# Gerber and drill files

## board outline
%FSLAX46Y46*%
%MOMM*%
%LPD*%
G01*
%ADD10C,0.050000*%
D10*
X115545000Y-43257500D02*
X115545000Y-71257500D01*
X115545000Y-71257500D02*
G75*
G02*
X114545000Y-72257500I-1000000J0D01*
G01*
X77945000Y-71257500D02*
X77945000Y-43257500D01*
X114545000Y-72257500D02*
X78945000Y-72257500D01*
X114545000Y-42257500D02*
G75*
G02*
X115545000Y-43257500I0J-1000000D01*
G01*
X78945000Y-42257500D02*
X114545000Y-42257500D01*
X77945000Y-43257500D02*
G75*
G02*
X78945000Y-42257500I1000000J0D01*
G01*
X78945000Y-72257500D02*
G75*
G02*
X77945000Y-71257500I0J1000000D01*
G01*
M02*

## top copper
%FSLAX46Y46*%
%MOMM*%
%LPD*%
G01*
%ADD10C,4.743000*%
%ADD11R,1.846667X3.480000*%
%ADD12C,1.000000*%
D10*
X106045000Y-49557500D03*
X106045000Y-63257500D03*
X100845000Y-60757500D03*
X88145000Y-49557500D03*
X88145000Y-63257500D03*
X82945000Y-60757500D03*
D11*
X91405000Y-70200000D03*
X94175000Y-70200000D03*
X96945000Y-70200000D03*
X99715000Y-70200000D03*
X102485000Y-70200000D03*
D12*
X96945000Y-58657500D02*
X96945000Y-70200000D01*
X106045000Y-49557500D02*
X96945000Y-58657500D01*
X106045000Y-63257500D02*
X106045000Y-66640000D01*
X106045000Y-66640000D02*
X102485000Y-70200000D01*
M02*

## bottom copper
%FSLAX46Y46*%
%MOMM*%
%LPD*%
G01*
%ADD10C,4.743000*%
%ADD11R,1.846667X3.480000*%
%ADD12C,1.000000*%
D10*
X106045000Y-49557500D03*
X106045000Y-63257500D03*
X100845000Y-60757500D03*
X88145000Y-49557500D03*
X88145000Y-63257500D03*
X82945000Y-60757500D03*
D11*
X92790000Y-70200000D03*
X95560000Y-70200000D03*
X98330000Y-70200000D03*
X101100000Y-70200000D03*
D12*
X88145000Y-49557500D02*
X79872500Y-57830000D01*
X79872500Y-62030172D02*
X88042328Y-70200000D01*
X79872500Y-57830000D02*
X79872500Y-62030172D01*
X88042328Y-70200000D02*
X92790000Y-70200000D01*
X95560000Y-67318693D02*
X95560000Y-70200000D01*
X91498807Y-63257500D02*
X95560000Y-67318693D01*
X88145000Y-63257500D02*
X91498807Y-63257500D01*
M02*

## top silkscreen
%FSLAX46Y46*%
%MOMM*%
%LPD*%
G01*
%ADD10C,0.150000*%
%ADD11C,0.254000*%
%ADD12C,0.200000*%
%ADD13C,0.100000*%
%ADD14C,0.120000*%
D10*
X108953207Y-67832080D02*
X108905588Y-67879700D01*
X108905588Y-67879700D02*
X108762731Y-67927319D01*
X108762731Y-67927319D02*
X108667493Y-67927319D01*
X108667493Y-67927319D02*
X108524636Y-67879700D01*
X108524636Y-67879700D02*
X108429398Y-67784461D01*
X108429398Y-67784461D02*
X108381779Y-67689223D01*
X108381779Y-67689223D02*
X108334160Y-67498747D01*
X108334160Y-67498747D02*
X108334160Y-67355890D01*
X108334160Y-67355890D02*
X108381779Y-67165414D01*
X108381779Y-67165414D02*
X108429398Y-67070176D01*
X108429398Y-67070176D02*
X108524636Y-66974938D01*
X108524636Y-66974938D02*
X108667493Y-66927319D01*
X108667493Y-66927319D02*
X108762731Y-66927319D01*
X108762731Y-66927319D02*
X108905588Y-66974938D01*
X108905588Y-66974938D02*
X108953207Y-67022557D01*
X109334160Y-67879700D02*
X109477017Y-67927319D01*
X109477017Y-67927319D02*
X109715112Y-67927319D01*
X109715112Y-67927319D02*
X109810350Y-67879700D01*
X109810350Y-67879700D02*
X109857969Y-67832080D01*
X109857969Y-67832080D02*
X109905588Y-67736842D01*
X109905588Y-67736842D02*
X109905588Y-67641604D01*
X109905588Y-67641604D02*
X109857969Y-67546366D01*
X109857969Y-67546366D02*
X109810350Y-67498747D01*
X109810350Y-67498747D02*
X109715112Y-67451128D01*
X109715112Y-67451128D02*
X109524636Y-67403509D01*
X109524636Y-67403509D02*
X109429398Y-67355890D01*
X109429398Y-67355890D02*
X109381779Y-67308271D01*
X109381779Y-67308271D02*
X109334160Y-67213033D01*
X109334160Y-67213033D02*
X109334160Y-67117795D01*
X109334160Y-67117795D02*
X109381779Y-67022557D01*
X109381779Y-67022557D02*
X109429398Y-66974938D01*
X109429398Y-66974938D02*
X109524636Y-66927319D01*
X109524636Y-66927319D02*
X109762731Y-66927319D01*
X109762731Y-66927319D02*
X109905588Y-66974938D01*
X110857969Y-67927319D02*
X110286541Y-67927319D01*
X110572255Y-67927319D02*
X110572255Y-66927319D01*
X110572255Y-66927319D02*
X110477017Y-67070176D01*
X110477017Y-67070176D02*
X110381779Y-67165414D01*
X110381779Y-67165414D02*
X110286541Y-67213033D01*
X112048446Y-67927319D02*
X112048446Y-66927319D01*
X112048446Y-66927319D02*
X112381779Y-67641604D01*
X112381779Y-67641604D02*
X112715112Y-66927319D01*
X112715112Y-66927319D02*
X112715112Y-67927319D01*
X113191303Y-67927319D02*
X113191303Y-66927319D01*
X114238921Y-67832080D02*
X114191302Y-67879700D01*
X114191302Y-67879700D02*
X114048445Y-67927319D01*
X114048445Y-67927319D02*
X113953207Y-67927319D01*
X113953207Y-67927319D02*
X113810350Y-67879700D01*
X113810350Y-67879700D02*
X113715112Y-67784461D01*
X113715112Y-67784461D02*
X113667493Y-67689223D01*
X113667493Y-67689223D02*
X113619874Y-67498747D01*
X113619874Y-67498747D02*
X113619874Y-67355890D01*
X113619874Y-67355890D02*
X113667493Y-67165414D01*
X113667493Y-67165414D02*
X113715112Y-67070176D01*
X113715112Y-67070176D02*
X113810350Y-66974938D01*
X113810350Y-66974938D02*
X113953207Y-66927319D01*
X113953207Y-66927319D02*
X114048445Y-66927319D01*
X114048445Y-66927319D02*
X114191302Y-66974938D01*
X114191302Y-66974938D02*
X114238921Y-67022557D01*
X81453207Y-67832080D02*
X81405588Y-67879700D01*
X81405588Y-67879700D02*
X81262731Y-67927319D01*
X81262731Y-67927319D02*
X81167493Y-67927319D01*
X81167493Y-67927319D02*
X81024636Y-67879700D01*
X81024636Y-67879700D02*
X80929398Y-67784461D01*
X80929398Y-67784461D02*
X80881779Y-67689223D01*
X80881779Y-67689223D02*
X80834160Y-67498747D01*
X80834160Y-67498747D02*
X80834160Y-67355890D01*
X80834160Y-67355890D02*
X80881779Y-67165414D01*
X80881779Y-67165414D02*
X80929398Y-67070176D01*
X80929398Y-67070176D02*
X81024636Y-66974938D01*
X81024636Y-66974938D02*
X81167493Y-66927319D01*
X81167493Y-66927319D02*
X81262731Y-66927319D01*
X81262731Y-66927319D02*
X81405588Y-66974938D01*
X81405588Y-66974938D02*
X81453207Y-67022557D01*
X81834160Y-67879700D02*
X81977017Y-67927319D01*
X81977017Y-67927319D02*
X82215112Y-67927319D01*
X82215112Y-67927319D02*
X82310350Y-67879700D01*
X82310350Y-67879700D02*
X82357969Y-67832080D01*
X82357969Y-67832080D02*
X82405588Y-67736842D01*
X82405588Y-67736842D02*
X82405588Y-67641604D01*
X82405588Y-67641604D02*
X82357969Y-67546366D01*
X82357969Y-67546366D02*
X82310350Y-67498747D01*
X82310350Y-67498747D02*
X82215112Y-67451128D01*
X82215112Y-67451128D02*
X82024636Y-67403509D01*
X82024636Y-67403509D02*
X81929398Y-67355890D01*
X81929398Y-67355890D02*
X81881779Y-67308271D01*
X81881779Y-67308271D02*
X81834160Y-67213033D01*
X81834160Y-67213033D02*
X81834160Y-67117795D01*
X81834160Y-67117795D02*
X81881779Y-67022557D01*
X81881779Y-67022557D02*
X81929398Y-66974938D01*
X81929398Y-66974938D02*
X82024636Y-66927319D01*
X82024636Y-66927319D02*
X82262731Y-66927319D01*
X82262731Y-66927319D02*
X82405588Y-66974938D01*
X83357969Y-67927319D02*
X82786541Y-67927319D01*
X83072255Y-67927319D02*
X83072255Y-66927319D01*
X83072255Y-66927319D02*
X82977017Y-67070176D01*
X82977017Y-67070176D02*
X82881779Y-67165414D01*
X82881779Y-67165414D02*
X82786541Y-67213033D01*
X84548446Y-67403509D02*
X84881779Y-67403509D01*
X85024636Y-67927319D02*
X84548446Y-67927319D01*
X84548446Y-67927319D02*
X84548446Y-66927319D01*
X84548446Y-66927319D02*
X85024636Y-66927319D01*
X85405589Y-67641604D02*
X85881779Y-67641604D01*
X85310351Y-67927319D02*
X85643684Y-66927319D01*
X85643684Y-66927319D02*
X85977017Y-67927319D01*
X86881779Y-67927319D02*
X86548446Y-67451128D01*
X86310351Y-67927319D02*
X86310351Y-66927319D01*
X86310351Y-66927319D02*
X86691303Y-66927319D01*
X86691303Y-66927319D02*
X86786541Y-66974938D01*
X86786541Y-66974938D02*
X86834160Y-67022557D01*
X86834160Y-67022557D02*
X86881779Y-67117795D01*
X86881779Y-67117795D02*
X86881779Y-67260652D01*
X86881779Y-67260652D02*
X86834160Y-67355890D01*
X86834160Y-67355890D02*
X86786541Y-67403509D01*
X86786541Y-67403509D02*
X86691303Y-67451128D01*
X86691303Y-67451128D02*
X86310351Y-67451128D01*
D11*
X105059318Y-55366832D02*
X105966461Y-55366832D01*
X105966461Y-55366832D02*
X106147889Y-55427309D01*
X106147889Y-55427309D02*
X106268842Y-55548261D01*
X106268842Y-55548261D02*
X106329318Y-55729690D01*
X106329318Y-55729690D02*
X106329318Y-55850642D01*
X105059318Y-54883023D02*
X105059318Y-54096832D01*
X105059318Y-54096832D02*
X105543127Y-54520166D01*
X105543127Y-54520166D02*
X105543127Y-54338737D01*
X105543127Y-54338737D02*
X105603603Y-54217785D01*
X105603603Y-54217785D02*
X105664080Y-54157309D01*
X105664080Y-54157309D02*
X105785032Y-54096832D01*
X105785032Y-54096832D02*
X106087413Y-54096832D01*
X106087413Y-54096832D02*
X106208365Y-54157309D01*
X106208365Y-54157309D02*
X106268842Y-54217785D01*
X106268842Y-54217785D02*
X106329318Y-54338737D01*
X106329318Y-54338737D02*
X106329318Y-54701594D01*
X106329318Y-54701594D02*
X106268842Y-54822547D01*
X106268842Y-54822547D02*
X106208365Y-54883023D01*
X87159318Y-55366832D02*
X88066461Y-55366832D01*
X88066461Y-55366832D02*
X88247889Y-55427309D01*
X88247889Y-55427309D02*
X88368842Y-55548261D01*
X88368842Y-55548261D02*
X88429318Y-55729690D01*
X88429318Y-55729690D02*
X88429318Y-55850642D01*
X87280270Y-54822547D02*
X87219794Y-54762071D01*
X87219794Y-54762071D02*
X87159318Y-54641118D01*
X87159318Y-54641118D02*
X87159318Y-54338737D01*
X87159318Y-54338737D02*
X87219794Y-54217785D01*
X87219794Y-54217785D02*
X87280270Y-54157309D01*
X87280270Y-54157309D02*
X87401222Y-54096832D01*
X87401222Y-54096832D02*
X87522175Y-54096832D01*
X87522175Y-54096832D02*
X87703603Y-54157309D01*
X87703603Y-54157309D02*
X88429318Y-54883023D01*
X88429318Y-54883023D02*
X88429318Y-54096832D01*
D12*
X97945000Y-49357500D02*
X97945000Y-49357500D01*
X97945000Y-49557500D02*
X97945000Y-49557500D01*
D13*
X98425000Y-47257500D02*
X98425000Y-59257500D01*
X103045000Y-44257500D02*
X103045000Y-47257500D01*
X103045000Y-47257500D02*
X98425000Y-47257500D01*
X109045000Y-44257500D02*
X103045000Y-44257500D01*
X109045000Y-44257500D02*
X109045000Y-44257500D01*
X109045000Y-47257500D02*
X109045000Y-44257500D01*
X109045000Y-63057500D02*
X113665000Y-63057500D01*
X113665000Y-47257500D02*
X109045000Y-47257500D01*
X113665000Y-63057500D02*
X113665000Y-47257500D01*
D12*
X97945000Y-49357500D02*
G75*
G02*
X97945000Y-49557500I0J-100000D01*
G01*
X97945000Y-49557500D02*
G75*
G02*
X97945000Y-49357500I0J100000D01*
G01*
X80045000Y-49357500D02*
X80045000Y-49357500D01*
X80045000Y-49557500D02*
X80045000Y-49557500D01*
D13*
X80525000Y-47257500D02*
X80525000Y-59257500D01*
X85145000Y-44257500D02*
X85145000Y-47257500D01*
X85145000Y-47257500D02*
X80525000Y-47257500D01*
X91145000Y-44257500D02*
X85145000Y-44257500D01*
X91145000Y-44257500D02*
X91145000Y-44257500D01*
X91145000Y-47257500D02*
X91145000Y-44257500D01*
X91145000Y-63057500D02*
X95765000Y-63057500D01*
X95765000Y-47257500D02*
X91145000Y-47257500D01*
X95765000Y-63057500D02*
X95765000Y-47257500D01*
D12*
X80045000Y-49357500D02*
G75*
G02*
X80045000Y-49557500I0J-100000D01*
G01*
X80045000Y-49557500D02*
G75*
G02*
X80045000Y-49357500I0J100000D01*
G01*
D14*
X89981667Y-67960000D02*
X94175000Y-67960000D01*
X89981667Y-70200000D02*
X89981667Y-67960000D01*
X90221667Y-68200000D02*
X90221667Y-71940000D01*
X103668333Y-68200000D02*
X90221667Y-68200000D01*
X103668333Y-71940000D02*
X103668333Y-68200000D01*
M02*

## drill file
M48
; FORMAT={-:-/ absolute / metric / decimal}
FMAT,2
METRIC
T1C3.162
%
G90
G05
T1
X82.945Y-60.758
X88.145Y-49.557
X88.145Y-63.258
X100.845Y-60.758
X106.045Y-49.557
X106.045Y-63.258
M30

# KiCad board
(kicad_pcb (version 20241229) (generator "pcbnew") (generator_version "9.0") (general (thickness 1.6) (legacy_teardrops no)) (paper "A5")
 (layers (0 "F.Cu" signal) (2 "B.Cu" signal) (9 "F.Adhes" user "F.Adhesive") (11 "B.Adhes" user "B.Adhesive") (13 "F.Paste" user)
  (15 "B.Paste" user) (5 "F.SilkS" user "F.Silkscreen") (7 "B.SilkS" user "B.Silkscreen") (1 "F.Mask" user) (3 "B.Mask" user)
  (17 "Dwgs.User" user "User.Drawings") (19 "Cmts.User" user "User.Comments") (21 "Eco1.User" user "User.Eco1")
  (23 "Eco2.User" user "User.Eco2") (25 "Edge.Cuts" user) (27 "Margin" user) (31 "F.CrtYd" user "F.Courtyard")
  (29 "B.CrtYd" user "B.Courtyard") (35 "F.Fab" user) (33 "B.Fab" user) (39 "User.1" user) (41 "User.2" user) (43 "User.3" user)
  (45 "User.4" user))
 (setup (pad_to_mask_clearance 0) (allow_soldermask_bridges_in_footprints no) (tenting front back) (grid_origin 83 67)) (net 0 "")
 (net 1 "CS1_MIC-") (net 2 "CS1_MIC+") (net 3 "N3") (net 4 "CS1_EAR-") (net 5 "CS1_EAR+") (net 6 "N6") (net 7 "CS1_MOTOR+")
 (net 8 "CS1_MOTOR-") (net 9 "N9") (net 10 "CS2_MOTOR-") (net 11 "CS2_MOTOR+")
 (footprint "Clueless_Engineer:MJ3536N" (layer "F.Cu") (at 105.755 54.9435 -90)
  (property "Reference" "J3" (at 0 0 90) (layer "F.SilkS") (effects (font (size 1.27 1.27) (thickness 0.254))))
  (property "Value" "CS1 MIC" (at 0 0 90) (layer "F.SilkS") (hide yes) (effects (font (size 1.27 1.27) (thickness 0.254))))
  (fp_line (start -5.586 7.81) (end -5.586 7.81) (stroke (width 0.2) (type solid)) (layer "F.SilkS"))
  (fp_line (start -5.386 7.81) (end -5.386 7.81) (stroke (width 0.2) (type solid)) (layer "F.SilkS"))
  (fp_line (start -7.686 7.33) (end 4.314 7.33) (stroke (width 0.1) (type solid)) (layer "F.SilkS"))
  (fp_line (start -10.686 2.71) (end -7.686 2.71) (stroke (width 0.1) (type solid)) (layer "F.SilkS"))
  (fp_line (start -7.686 2.71) (end -7.686 7.33) (stroke (width 0.1) (type solid)) (layer "F.SilkS"))
  (fp_line (start -10.686 -3.29) (end -10.686 2.71) (stroke (width 0.1) (type solid)) (layer "F.SilkS"))
  (fp_line (start -10.686 -3.29) (end -10.686 -3.29) (stroke (width 0.1) (type solid)) (layer "F.SilkS"))
  (fp_line (start -7.686 -3.29) (end -10.686 -3.29) (stroke (width 0.1) (type solid)) (layer "F.SilkS"))
  (fp_line (start 8.114 -3.29) (end 8.114 -7.91) (stroke (width 0.1) (type solid)) (layer "F.SilkS"))
  (fp_line (start -7.686 -7.91) (end -7.686 -3.29) (stroke (width 0.1) (type solid)) (layer "F.SilkS"))
  (fp_line (start 8.114 -7.91) (end -7.686 -7.91) (stroke (width 0.1) (type solid)) (layer "F.SilkS"))
  (fp_arc (start -5.586 7.81) (mid -5.486 7.71) (end -5.386 7.81) (stroke (width 0.2) (type solid)) (layer "F.SilkS"))
  (fp_arc (start -5.386 7.81) (mid -5.486 7.91) (end -5.586 7.81) (stroke (width 0.2) (type solid)) (layer "F.SilkS"))
  (pad "1" thru_hole circle (at -5.386 -0.29 270) (size 4.743 4.743) (drill 3.1623) (layers "*.Cu" "*.Mask") (remove_unused_layers no)
   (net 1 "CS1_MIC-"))
  (pad "2" thru_hole circle (at 8.314 -0.29 270) (size 4.743 4.743) (drill 3.1623) (layers "*.Cu" "*.Mask") (remove_unused_layers no)
   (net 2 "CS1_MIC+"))
  (pad "3" thru_hole circle (at 5.814 4.91 270) (size 4.743 4.743) (drill 3.1623) (layers "*.Cu" "*.Mask") (remove_unused_layers no)
   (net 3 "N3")))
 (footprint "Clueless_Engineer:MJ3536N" (layer "F.Cu") (at 87.855 54.9435 -90)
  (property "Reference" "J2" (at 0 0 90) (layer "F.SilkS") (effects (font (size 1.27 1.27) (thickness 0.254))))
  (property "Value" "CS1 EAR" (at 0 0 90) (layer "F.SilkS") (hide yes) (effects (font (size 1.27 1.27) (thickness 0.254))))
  (fp_line (start -5.586 7.81) (end -5.586 7.81) (stroke (width 0.2) (type solid)) (layer "F.SilkS"))
  (fp_line (start -5.386 7.81) (end -5.386 7.81) (stroke (width 0.2) (type solid)) (layer "F.SilkS"))
  (fp_line (start -7.686 7.33) (end 4.314 7.33) (stroke (width 0.1) (type solid)) (layer "F.SilkS"))
  (fp_line (start -10.686 2.71) (end -7.686 2.71) (stroke (width 0.1) (type solid)) (layer "F.SilkS"))
  (fp_line (start -7.686 2.71) (end -7.686 7.33) (stroke (width 0.1) (type solid)) (layer "F.SilkS"))
  (fp_line (start -10.686 -3.29) (end -10.686 2.71) (stroke (width 0.1) (type solid)) (layer "F.SilkS"))
  (fp_line (start -10.686 -3.29) (end -10.686 -3.29) (stroke (width 0.1) (type solid)) (layer "F.SilkS"))
  (fp_line (start -7.686 -3.29) (end -10.686 -3.29) (stroke (width 0.1) (type solid)) (layer "F.SilkS"))
  (fp_line (start 8.114 -3.29) (end 8.114 -7.91) (stroke (width 0.1) (type solid)) (layer "F.SilkS"))
  (fp_line (start -7.686 -7.91) (end -7.686 -3.29) (stroke (width 0.1) (type solid)) (layer "F.SilkS"))
  (fp_line (start 8.114 -7.91) (end -7.686 -7.91) (stroke (width 0.1) (type solid)) (layer "F.SilkS"))
  (fp_arc (start -5.586 7.81) (mid -5.486 7.71) (end -5.386 7.81) (stroke (width 0.2) (type solid)) (layer "F.SilkS"))
  (fp_arc (start -5.386 7.81) (mid -5.486 7.91) (end -5.586 7.81) (stroke (width 0.2) (type solid)) (layer "F.SilkS"))
  (pad "1" thru_hole circle (at -5.386 -0.29 270) (size 4.743 4.743) (drill 3.1623) (layers "*.Cu" "*.Mask") (remove_unused_layers no)
   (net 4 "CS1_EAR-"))
  (pad "2" thru_hole circle (at 8.314 -0.29 270) (size 4.743 4.743) (drill 3.1623) (layers "*.Cu" "*.Mask") (remove_unused_layers no)
   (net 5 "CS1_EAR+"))
  (pad "3" thru_hole circle (at 5.814 4.91 270) (size 4.743 4.743) (drill 3.1623) (layers "*.Cu" "*.Mask") (remove_unused_layers no)
   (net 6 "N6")))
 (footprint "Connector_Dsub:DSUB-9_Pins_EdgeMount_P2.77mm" (layer "F.Cu") (at 96.945 70.2)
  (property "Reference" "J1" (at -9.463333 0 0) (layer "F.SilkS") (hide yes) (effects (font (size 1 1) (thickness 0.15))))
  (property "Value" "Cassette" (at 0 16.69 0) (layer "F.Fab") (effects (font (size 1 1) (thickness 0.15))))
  (fp_line (start -6.963333 -2.24) (end -2.77 -2.24) (stroke (width 0.12) (type solid)) (layer "F.SilkS"))
  (fp_line (start -6.963333 0) (end -6.963333 -2.24) (stroke (width 0.12) (type solid)) (layer "F.SilkS"))
  (fp_line (start -6.723333 -2) (end -6.723333 1.74) (stroke (width 0.12) (type solid)) (layer "F.SilkS"))
  (fp_line (start 6.723333 -2) (end -6.723333 -2) (stroke (width 0.12) (type solid)) (layer "F.SilkS"))
  (fp_line (start 6.723333 1.74) (end 6.723333 -2) (stroke (width 0.12) (type solid)) (layer "F.SilkS"))
  (pad "1" smd rect (at -5.54 0) (size 1.846667 3.48) (layers "F.Cu" "F.Mask" "F.Paste") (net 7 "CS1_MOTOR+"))
  (pad "2" smd rect (at -2.77 0) (size 1.846667 3.48) (layers "F.Cu" "F.Mask" "F.Paste") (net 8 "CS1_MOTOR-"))
  (pad "3" smd rect (at 0 0) (size 1.846667 3.48) (layers "F.Cu" "F.Mask" "F.Paste") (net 1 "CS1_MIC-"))
  (pad "4" smd rect (at 2.77 0) (size 1.846667 3.48) (layers "F.Cu" "F.Mask" "F.Paste") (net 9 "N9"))
  (pad "5" smd rect (at 5.54 0) (size 1.846667 3.48) (layers "F.Cu" "F.Mask" "F.Paste") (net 2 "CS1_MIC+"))
  (pad "6" smd rect (at -4.155 0) (size 1.846667 3.48) (layers "B.Cu" "B.Mask" "B.Paste") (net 4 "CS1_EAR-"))
  (pad "7" smd rect (at -1.385 0) (size 1.846667 3.48) (layers "B.Cu" "B.Mask" "B.Paste") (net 5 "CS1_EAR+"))
  (pad "8" smd rect (at 1.385 0) (size 1.846667 3.48) (layers "B.Cu" "B.Mask" "B.Paste") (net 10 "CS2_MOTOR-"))
  (pad "9" smd rect (at 4.155 0) (size 1.846667 3.48) (layers "B.Cu" "B.Mask" "B.Paste") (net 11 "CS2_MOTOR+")))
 (gr_line (start 115.545 43.2575) (end 115.545 71.2575) (stroke (width 0.05) (type default)) (layer "Edge.Cuts"))
 (gr_arc (start 115.545 71.2575) (mid 115.252107 71.964607) (end 114.545 72.2575) (stroke (width 0.05) (type default)) (layer "Edge.Cuts"))
 (gr_line (start 77.945 71.2575) (end 77.945 43.2575) (stroke (width 0.05) (type default)) (layer "Edge.Cuts"))
 (gr_line (start 114.545 72.2575) (end 78.945 72.2575) (stroke (width 0.05) (type default)) (layer "Edge.Cuts"))
 (gr_arc (start 114.545 42.2575) (mid 115.252107 42.550393) (end 115.545 43.2575) (stroke (width 0.05) (type default)) (layer "Edge.Cuts"))
 (gr_line (start 78.945 42.2575) (end 114.545 42.2575) (stroke (width 0.05) (type default)) (layer "Edge.Cuts"))
 (gr_arc (start 77.945 43.2575) (mid 78.237893 42.550393) (end 78.945 42.2575) (stroke (width 0.05) (type default)) (layer "Edge.Cuts"))
 (gr_arc (start 78.945 72.2575) (mid 78.237893 71.964607) (end 77.945 71.2575) (stroke (width 0.05) (type default)) (layer "Edge.Cuts"))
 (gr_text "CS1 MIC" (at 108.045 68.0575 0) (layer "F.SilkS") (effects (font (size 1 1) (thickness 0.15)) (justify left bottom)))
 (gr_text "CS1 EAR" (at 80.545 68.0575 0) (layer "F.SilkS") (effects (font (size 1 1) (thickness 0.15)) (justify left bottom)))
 (segment (start 96.945 58.6575) (end 96.945 70.2) (width 1) (layer "F.Cu") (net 1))
 (segment (start 106.045 49.5575) (end 96.945 58.6575) (width 1) (layer "F.Cu") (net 1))
 (segment (start 106.045 63.2575) (end 106.045 66.64) (width 1) (layer "F.Cu") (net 2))
 (segment (start 106.045 66.64) (end 102.485 70.2) (width 1) (layer "F.Cu") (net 2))
 (segment (start 88.145 49.5575) (end 79.8725 57.83) (width 1) (layer "B.Cu") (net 4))
 (segment (start 79.8725 62.030172) (end 88.042328 70.2) (width 1) (layer "B.Cu") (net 4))
 (segment (start 79.8725 57.83) (end 79.8725 62.030172) (width 1) (layer "B.Cu") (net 4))
 (segment (start 88.042328 70.2) (end 92.79 70.2) (width 1) (layer "B.Cu") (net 4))
 (segment (start 95.56 67.318693) (end 95.56 70.2) (width 1) (layer "B.Cu") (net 5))
 (segment (start 91.498807 63.2575) (end 95.56 67.318693) (width 1) (layer "B.Cu") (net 5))
 (segment (start 88.145 63.2575) (end 91.498807 63.2575) (width 1) (layer "B.Cu") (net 5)))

